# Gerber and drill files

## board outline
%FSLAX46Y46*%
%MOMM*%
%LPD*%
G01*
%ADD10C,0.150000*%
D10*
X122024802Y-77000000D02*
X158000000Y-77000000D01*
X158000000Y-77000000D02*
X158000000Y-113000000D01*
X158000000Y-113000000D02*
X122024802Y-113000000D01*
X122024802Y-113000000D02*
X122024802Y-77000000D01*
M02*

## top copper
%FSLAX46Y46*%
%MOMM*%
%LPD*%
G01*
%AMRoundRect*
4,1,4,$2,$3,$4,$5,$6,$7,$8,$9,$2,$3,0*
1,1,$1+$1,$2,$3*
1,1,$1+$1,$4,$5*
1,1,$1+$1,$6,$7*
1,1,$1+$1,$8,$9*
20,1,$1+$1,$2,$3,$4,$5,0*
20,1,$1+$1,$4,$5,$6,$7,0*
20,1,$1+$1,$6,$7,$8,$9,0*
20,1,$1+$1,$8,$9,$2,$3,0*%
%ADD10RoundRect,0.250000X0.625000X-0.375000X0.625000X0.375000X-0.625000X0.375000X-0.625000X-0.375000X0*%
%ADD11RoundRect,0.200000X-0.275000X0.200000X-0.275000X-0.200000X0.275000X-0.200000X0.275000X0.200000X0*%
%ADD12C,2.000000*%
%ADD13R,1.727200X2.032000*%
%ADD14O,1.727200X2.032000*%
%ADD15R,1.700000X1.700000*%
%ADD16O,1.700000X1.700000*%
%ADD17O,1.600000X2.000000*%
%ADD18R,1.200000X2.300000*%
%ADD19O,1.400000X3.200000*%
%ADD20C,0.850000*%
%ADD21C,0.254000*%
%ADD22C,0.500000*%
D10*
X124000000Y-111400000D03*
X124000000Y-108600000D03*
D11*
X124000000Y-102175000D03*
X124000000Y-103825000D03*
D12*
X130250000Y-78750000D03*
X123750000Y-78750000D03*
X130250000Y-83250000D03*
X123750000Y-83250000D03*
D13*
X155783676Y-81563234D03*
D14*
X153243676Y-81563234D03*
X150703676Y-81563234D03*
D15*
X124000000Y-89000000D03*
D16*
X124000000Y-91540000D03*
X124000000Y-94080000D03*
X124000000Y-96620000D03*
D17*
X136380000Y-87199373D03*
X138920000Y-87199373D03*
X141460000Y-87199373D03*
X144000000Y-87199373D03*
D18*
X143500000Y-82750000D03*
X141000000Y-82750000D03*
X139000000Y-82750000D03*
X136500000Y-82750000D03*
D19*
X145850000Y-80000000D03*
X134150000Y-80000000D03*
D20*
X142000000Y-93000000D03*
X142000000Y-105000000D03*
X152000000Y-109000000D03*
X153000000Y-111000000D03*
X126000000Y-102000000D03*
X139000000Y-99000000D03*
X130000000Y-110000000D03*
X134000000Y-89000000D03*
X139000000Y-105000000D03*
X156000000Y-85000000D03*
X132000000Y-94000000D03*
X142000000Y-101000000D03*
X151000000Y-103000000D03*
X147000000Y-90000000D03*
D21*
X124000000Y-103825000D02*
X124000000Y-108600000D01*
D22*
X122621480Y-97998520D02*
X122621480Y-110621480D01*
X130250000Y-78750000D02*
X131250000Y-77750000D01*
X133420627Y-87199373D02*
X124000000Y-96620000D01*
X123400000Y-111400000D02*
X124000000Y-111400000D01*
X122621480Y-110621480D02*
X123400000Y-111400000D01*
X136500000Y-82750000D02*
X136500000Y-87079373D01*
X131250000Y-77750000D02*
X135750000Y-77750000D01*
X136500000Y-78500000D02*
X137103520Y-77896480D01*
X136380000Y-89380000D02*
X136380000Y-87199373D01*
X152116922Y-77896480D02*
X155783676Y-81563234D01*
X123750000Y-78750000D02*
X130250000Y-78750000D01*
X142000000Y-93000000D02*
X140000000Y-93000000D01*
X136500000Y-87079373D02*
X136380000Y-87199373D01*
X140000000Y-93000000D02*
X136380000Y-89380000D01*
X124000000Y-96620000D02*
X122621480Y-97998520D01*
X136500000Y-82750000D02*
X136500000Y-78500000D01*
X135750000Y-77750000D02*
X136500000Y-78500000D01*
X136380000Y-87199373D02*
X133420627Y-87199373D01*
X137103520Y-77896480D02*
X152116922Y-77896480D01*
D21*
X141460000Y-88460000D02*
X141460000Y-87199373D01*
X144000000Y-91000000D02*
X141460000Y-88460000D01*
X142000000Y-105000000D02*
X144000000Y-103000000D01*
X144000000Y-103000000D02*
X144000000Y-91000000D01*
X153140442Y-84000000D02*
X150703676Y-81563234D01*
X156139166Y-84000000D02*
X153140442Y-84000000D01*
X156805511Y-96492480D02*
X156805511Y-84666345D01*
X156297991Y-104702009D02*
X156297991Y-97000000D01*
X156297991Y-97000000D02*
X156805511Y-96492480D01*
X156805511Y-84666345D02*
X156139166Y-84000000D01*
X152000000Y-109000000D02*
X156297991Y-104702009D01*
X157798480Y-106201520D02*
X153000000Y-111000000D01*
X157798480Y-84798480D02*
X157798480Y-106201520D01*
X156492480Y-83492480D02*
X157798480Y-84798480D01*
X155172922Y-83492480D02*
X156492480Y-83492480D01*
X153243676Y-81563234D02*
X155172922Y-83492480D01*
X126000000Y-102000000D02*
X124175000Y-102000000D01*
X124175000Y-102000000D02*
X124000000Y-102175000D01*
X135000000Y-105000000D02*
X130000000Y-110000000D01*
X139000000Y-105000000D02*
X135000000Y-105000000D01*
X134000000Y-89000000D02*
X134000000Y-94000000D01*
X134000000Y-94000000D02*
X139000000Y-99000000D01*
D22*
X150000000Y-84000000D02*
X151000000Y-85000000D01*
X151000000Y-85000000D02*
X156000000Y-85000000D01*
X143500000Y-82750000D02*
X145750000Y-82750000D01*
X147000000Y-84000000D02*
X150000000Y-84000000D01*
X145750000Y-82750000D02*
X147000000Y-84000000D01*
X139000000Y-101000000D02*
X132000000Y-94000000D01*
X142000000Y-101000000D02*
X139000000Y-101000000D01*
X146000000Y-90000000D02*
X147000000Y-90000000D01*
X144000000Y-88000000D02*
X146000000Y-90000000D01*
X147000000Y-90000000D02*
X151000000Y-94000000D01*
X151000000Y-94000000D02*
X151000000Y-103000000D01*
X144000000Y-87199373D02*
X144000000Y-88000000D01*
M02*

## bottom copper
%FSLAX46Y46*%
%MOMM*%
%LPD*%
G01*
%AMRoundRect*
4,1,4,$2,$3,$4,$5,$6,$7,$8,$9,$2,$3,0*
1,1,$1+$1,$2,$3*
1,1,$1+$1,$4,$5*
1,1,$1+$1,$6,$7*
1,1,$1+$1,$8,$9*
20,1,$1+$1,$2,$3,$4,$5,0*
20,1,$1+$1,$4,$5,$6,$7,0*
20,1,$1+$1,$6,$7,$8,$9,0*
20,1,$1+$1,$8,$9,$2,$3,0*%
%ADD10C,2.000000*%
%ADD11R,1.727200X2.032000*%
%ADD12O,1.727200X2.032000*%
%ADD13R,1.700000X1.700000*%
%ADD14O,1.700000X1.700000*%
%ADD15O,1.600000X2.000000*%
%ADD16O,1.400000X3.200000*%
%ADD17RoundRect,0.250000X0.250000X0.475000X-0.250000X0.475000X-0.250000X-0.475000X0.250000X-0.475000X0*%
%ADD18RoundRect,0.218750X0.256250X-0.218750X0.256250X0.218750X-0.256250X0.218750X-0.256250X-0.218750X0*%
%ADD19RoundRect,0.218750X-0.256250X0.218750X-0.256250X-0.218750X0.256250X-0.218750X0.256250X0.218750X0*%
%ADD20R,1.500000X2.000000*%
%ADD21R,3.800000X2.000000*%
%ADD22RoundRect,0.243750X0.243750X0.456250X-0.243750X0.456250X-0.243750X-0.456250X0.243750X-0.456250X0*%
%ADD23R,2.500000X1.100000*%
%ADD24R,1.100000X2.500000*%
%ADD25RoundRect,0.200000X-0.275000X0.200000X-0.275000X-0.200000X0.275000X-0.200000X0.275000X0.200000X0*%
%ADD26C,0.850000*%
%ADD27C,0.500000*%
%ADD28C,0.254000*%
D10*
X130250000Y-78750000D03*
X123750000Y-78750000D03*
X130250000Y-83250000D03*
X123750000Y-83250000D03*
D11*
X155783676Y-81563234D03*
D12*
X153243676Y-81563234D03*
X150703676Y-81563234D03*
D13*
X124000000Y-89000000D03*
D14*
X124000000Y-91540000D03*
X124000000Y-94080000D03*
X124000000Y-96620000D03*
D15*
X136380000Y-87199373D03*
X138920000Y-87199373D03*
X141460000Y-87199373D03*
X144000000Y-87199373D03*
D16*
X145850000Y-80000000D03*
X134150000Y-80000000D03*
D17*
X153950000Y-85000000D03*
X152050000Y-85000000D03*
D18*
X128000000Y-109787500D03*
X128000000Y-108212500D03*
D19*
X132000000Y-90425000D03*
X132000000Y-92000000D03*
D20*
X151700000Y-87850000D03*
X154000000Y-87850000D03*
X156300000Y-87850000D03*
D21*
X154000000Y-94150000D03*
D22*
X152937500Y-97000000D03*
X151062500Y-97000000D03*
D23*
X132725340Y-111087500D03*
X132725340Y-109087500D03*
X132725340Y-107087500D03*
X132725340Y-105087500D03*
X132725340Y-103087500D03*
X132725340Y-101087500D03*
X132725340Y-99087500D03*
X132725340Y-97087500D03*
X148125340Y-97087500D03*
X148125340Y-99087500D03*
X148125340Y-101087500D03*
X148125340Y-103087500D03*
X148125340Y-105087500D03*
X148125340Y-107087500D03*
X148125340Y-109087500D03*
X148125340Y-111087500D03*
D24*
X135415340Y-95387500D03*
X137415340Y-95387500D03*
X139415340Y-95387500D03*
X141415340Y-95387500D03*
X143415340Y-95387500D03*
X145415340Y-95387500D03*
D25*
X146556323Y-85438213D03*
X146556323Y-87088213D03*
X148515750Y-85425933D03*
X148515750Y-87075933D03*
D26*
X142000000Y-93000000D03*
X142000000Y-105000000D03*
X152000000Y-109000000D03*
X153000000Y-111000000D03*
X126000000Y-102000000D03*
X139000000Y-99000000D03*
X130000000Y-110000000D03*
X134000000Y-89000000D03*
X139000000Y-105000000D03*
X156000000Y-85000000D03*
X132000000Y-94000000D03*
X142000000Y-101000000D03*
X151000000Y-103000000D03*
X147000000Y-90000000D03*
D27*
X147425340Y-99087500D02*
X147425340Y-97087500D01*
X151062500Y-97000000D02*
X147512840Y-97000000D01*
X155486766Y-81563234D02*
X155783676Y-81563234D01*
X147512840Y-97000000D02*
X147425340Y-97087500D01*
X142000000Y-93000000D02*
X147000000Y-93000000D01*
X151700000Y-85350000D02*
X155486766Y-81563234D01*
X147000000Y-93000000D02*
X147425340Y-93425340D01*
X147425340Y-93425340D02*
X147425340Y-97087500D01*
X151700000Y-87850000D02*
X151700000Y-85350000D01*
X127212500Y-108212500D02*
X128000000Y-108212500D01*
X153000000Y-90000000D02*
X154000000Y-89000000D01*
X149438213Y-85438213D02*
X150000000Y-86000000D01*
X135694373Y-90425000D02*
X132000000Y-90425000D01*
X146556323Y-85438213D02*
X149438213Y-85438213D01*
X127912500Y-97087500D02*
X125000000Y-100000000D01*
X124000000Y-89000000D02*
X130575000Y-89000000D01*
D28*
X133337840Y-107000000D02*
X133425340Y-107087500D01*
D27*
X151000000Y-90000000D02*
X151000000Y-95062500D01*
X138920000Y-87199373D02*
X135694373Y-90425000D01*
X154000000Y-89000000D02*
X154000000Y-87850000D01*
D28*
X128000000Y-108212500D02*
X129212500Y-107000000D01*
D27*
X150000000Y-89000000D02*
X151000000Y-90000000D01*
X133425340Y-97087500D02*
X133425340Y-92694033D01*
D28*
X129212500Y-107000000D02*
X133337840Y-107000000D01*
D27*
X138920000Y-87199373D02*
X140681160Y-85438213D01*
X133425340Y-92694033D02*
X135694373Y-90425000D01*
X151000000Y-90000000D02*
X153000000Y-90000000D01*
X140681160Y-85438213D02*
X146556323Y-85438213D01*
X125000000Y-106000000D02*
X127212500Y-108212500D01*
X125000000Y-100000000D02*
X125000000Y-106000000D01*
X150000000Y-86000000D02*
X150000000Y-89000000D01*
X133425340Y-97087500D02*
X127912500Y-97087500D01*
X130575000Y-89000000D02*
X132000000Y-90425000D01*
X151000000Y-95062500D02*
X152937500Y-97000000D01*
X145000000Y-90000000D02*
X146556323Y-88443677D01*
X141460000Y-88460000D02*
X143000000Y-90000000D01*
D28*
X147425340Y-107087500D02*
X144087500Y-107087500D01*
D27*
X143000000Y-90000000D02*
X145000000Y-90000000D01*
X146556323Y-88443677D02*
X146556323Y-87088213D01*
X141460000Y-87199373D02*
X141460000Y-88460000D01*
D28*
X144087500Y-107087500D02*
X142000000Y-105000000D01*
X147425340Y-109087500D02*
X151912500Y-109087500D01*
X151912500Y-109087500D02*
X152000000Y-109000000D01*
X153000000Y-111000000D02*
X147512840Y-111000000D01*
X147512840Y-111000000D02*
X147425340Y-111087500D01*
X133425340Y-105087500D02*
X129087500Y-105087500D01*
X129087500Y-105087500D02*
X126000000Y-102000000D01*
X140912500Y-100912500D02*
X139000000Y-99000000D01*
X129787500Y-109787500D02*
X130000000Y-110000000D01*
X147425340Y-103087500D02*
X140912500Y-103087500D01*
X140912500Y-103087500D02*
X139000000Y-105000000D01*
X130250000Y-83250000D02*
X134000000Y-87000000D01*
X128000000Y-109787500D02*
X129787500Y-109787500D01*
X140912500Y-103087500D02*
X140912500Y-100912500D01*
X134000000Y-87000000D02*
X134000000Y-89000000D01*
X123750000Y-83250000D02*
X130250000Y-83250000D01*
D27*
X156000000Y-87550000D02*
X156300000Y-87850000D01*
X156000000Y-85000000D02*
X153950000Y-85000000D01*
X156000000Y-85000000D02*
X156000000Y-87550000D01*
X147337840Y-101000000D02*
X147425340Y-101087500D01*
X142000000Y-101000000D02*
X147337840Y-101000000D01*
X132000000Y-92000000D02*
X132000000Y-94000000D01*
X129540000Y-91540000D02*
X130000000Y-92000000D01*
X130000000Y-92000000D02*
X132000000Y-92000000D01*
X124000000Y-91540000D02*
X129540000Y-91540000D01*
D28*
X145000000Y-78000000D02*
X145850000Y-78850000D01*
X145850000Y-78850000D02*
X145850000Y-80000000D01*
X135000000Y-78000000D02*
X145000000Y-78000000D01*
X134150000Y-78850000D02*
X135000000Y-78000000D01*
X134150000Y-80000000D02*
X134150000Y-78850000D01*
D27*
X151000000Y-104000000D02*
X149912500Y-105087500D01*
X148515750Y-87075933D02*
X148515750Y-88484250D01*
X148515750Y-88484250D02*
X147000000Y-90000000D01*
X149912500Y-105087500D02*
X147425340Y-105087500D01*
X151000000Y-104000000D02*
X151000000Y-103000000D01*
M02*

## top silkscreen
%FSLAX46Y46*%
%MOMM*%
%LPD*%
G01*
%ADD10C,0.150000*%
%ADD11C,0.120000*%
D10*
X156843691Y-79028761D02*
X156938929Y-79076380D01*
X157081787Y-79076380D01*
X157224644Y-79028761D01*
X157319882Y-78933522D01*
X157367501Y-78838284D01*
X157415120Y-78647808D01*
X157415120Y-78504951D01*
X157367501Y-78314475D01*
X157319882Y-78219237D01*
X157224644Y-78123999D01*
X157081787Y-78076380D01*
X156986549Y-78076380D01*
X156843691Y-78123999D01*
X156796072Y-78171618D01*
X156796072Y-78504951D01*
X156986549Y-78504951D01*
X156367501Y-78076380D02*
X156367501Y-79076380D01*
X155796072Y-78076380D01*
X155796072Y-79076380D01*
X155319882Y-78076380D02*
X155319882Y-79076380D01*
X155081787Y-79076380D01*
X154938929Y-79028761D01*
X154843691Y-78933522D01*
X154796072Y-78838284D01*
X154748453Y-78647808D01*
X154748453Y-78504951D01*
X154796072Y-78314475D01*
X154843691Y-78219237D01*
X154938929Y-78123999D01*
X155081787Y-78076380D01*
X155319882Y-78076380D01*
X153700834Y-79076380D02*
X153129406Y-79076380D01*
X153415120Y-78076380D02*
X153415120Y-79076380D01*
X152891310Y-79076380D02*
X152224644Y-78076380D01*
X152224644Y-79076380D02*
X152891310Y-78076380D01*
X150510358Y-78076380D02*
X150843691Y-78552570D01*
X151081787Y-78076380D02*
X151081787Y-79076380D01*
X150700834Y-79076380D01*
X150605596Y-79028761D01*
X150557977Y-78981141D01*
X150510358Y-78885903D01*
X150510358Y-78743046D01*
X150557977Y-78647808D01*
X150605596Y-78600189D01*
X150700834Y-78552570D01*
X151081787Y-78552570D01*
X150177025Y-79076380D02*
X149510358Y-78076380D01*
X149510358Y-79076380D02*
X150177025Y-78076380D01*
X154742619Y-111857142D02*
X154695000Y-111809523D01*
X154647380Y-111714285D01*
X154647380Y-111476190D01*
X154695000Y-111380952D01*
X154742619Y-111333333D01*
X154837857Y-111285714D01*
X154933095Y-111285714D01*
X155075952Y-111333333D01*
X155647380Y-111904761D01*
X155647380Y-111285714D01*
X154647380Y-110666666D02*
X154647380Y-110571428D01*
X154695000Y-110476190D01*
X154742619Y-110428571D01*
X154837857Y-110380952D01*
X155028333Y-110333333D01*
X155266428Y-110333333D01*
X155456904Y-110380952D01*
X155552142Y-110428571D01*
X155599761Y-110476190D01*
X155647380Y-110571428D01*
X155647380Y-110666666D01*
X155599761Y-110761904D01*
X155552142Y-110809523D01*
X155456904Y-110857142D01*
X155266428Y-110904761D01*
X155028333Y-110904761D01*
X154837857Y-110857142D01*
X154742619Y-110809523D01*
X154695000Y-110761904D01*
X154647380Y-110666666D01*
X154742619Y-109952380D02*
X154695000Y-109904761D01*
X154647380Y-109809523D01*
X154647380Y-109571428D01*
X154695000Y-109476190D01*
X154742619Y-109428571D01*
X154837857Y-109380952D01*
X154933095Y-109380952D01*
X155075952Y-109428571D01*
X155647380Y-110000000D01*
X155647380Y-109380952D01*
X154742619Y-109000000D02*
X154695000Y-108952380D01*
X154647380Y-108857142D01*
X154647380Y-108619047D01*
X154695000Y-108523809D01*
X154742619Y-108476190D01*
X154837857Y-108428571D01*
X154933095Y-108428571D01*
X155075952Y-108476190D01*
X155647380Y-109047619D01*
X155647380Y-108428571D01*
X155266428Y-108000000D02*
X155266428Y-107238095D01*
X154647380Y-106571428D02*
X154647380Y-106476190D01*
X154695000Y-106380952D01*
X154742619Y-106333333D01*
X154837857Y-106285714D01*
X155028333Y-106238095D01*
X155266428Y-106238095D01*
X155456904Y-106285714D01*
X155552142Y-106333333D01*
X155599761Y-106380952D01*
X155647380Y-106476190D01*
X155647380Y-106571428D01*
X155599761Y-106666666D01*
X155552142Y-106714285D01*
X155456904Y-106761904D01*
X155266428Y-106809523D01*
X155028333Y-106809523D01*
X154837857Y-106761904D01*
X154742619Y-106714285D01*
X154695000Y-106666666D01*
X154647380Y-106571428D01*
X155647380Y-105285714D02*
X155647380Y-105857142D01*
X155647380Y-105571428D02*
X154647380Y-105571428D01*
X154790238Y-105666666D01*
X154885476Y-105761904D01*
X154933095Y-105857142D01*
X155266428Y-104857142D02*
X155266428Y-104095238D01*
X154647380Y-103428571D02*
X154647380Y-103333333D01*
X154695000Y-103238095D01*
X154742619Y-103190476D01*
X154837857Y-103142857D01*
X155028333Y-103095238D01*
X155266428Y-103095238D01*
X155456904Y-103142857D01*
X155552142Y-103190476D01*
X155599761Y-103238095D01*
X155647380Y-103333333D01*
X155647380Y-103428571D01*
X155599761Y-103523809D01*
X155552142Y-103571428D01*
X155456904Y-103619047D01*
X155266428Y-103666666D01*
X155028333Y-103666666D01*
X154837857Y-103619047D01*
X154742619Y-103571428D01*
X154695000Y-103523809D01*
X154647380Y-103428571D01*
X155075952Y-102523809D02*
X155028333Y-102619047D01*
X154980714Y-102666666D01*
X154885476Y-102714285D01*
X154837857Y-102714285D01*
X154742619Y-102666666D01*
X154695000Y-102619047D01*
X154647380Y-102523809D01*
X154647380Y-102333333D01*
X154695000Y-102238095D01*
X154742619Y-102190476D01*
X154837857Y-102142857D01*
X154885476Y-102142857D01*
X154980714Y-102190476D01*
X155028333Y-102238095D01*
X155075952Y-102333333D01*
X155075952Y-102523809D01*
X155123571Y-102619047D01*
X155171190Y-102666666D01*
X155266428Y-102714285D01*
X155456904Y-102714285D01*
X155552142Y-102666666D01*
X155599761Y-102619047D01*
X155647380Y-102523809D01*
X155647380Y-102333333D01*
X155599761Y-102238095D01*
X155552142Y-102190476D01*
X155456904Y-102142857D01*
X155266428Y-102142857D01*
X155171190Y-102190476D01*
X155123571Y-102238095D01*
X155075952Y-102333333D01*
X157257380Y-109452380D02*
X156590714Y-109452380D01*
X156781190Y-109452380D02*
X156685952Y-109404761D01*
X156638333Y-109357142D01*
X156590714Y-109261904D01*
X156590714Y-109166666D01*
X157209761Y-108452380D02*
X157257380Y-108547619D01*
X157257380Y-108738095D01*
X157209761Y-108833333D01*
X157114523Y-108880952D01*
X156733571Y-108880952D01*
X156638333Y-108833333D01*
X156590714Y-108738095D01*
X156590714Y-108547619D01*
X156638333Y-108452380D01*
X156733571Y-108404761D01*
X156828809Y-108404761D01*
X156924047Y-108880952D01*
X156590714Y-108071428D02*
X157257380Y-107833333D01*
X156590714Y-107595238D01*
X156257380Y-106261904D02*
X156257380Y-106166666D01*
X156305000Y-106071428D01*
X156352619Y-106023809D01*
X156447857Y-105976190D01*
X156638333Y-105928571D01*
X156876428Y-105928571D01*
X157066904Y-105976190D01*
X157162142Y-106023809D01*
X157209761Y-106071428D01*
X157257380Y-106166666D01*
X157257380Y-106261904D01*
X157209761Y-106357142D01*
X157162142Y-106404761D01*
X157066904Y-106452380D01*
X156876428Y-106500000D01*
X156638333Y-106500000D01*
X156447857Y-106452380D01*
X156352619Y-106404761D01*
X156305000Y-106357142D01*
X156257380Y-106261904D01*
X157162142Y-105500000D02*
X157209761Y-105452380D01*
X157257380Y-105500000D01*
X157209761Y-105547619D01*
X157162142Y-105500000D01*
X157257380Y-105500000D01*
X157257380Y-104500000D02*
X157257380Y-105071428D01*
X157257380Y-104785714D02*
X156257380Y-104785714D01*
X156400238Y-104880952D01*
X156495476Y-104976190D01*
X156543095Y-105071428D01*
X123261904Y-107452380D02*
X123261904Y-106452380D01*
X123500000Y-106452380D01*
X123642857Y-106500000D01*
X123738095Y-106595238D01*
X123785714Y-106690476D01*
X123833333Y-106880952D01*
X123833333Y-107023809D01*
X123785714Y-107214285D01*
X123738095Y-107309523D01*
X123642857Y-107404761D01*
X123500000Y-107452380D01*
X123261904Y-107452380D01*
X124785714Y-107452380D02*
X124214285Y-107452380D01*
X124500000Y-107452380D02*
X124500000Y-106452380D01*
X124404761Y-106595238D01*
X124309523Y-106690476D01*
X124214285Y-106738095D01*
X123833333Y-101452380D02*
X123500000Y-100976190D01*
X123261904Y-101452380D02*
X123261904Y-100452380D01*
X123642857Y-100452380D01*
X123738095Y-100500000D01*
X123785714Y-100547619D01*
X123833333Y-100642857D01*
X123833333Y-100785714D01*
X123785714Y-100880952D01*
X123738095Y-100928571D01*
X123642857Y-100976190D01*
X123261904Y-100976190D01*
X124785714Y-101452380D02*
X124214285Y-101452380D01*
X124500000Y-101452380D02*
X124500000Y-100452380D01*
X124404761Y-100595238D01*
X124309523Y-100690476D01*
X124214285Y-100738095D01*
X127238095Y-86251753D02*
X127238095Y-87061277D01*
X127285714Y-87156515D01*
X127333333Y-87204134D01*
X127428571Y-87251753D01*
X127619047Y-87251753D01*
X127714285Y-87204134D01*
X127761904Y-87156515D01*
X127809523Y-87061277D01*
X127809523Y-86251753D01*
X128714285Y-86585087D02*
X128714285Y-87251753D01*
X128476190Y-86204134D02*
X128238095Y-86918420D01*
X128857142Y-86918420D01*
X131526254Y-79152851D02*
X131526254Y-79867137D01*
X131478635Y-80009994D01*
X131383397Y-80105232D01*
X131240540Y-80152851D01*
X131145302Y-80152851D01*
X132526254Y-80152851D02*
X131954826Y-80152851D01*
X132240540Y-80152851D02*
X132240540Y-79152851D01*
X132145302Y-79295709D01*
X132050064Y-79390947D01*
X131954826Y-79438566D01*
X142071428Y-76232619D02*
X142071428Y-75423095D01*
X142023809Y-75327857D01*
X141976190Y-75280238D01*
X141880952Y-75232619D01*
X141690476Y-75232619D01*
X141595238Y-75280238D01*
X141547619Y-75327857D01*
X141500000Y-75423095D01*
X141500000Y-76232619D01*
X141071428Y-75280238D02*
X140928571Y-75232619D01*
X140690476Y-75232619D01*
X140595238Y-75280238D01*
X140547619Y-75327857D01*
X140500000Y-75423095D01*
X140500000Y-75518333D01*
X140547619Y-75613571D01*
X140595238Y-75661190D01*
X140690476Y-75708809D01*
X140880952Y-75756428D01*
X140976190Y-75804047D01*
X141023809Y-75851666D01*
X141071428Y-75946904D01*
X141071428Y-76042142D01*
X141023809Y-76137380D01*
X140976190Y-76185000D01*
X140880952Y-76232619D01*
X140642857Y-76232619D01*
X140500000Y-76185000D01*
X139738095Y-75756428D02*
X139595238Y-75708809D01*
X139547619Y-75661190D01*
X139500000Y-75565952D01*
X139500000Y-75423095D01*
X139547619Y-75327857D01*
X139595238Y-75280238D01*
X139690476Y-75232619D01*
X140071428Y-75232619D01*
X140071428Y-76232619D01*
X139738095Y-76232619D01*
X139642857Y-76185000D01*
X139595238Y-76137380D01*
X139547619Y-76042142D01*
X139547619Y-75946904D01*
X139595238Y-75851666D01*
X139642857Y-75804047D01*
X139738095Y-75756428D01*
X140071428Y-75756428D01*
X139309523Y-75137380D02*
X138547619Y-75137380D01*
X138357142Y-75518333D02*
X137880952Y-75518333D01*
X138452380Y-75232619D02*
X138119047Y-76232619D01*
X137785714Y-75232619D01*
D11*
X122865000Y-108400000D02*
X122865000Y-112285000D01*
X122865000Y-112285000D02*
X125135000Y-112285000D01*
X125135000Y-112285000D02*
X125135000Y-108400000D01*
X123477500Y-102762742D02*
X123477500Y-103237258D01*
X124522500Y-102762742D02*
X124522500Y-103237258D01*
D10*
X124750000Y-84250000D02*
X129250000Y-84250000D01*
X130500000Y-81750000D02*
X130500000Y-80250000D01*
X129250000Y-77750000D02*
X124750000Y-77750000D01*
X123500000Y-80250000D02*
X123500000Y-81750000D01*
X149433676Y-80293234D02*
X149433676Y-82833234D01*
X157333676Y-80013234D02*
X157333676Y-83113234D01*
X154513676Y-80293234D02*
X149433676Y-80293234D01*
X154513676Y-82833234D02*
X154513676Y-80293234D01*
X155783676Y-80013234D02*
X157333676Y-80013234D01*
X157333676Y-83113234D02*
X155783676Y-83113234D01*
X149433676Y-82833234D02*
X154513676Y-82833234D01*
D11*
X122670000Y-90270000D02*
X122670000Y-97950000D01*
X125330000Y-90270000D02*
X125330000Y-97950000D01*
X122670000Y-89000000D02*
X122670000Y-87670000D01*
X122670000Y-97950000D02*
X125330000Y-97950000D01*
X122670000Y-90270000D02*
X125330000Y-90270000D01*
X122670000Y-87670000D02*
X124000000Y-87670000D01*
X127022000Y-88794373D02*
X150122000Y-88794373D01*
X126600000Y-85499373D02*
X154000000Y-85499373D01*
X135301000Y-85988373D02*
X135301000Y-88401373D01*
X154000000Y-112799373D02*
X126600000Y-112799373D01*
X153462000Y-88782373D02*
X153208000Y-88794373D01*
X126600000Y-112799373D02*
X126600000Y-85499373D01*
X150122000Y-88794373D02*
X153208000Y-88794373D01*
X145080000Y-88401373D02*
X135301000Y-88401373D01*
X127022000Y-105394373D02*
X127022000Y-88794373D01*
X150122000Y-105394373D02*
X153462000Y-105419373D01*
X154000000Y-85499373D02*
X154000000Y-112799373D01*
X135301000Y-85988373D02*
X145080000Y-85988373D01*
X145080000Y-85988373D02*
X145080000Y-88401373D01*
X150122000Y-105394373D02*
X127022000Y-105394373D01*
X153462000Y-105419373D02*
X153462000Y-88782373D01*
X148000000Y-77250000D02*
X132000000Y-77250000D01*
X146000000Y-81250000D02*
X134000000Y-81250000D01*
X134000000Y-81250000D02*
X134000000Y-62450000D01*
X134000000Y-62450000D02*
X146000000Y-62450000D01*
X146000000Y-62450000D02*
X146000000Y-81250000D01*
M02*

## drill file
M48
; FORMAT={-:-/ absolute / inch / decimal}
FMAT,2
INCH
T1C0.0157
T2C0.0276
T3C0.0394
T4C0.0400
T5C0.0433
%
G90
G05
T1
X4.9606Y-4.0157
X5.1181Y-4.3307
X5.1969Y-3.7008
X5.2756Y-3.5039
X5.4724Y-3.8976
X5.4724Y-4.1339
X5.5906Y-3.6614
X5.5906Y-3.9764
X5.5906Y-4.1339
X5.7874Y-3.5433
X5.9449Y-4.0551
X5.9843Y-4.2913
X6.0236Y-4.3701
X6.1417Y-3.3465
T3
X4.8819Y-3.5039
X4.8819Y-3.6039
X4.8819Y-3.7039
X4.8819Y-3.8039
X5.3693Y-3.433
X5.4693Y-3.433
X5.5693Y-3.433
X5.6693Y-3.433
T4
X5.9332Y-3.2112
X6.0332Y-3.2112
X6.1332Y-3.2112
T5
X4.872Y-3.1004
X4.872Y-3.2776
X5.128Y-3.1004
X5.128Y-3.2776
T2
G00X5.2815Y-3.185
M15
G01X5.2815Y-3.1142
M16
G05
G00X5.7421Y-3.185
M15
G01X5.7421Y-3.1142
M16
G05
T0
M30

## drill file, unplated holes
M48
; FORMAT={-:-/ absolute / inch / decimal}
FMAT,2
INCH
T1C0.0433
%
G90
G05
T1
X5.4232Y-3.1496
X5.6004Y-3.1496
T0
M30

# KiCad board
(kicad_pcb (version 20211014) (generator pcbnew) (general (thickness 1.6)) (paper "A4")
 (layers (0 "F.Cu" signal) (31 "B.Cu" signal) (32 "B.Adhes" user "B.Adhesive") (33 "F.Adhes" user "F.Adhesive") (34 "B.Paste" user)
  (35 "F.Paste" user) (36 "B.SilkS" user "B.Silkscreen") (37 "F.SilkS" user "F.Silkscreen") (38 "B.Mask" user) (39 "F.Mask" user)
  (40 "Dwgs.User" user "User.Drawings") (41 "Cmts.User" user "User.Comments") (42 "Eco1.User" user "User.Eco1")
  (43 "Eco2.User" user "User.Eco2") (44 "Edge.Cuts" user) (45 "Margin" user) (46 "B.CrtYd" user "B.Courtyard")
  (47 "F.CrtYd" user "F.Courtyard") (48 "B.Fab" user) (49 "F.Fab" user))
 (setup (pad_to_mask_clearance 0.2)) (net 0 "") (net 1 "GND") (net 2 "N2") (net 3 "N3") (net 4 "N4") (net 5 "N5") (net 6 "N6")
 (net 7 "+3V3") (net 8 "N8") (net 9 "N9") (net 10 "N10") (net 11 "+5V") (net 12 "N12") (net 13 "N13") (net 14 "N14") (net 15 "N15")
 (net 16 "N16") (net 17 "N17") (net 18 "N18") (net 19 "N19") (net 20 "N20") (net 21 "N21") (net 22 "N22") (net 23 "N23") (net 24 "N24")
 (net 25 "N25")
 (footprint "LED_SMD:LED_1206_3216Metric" (layer "F.Cu") (at 124 110 90)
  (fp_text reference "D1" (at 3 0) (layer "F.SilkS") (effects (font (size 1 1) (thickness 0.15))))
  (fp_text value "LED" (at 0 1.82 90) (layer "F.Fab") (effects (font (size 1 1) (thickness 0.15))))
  (fp_line (start 1.6 -1.135) (end -2.285 -1.135) (layer "F.SilkS") (width 0.12))
  (fp_line (start -2.285 -1.135) (end -2.285 1.135) (layer "F.SilkS") (width 0.12))
  (fp_line (start -2.285 1.135) (end 1.6 1.135) (layer "F.SilkS") (width 0.12))
  (pad "1" smd roundrect locked (at -1.4 0 90) (size 1.25 1.75) (layers "F.Cu" "F.Paste" "F.Mask") (roundrect_rratio 0.2) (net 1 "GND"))
  (pad "2" smd roundrect locked (at 1.4 0 90) (size 1.25 1.75) (layers "F.Cu" "F.Paste" "F.Mask") (roundrect_rratio 0.2) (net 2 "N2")))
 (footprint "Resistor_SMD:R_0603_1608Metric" (layer "F.Cu") (at 124 103 -90)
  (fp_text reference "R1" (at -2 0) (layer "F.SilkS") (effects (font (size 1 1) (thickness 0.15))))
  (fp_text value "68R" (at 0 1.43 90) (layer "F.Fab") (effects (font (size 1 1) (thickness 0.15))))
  (fp_line (start -0.237258 0.5225) (end 0.237258 0.5225) (layer "F.SilkS") (width 0.12))
  (fp_line (start -0.237258 -0.5225) (end 0.237258 -0.5225) (layer "F.SilkS") (width 0.12))
  (pad "1" smd roundrect locked (at -0.825 0 270) (size 0.8 0.95) (layers "F.Cu" "F.Paste" "F.Mask") (roundrect_rratio 0.25) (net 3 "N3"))
  (pad "2" smd roundrect locked (at 0.825 0 270) (size 0.8 0.95) (layers "F.Cu" "F.Paste" "F.Mask") (roundrect_rratio 0.25) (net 2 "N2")))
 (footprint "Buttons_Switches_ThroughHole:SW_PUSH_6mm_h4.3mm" (layer "F.Cu") (at 123.75 78.75)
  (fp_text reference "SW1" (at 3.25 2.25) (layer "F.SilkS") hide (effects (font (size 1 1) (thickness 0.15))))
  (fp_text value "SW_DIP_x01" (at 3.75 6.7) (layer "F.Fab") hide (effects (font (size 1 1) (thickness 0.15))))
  (fp_line (start 1 5.5) (end 5.5 5.5) (layer "F.SilkS") (width 0.15))
  (fp_line (start 6.75 3) (end 6.75 1.5) (layer "F.SilkS") (width 0.15))
  (fp_line (start 5.5 -1) (end 1 -1) (layer "F.SilkS") (width 0.15))
  (fp_line (start -0.25 1.5) (end -0.25 3) (layer "F.SilkS") (width 0.15))
  (pad "1" thru_hole circle locked (at 6.5 0 90) (size 2 2) (drill 1.1) (layers *.Cu *.Mask) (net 1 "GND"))
  (pad "1" thru_hole circle locked (at 0 0 90) (size 2 2) (drill 1.1) (layers *.Cu *.Mask) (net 1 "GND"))
  (pad "2" thru_hole circle locked (at 6.5 4.5 90) (size 2 2) (drill 1.1) (layers *.Cu *.Mask) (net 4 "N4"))
  (pad "2" thru_hole circle locked (at 0 4.5 90) (size 2 2) (drill 1.1) (layers *.Cu *.Mask) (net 4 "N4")))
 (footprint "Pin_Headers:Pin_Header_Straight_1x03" (layer "F.Cu") (at 155.783676 81.563234 -90)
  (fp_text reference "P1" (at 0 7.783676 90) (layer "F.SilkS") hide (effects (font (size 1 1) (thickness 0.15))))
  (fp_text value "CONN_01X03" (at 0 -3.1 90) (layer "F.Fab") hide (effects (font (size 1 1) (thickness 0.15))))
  (fp_line (start -1.27 6.35) (end 1.27 6.35) (layer "F.SilkS") (width 0.15))
  (fp_line (start -1.55 -1.55) (end 1.55 -1.55) (layer "F.SilkS") (width 0.15))
  (fp_line (start -1.27 1.27) (end -1.27 6.35) (layer "F.SilkS") (width 0.15))
  (fp_line (start 1.27 1.27) (end -1.27 1.27) (layer "F.SilkS") (width 0.15))
  (fp_line (start -1.55 0) (end -1.55 -1.55) (layer "F.SilkS") (width 0.15))
  (fp_line (start 1.55 -1.55) (end 1.55 0) (layer "F.SilkS") (width 0.15))
  (fp_line (start 1.27 6.35) (end 1.27 1.27) (layer "F.SilkS") (width 0.15))
  (pad "1" thru_hole rect locked (at 0 0 270) (size 2.032 1.7272) (drill 1.016) (layers *.Cu *.Mask) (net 1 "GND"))
  (pad "2" thru_hole oval locked (at 0 2.54 270) (size 2.032 1.7272) (drill 1.016) (layers *.Cu *.Mask) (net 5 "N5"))
  (pad "3" thru_hole oval locked (at 0 5.08 270) (size 2.032 1.7272) (drill 1.016) (layers *.Cu *.Mask) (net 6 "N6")))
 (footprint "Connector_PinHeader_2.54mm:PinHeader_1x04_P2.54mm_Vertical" (layer "F.Cu") (at 124 89)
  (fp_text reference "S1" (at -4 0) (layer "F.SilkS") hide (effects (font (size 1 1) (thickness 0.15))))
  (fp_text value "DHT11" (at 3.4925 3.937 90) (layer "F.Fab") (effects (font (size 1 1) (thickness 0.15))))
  (fp_line (start -1.33 1.27) (end -1.33 8.95) (layer "F.SilkS") (width 0.12))
  (fp_line (start 1.33 1.27) (end 1.33 8.95) (layer "F.SilkS") (width 0.12))
  (fp_line (start -1.33 0) (end -1.33 -1.33) (layer "F.SilkS") (width 0.12))
  (fp_line (start -1.33 8.95) (end 1.33 8.95) (layer "F.SilkS") (width 0.12))
  (fp_line (start -1.33 1.27) (end 1.33 1.27) (layer "F.SilkS") (width 0.12))
  (fp_line (start -1.33 -1.33) (end 0 -1.33) (layer "F.SilkS") (width 0.12))
  (pad "1" thru_hole rect locked (at 0 0) (size 1.7 1.7) (drill 1) (layers *.Cu *.Mask) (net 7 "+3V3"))
  (pad "2" thru_hole oval locked (at 0 2.54) (size 1.7 1.7) (drill 1) (layers *.Cu *.Mask) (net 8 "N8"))
  (pad "3" thru_hole oval locked (at 0 5.08) (size 1.7 1.7) (drill 1) (layers *.Cu *.Mask))
  (pad "4" thru_hole oval locked (at 0 7.62) (size 1.7 1.7) (drill 1) (layers *.Cu *.Mask) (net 1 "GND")))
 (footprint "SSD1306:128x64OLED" (layer "F.Cu") (at 140 97.799373)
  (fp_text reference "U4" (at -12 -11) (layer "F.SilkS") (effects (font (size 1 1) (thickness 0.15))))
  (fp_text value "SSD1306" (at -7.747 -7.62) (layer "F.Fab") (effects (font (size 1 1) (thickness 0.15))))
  (fp_line (start -12.978 -9.005) (end 10.122 -9.005) (layer "F.SilkS") (width 0.12))
  (fp_line (start -13.4 -12.3) (end 14 -12.3) (layer "F.SilkS") (width 0.12))
  (fp_line (start -4.699 -11.811) (end -4.699 -9.398) (layer "F.SilkS") (width 0.12))
  (fp_line (start 14 15) (end -13.4 15) (layer "F.SilkS") (width 0.12))
  (fp_line (start 13.462 -9.017) (end 13.208 -9.005) (layer "F.SilkS") (width 0.12))
  (fp_line (start -13.4 15) (end -13.4 -12.3) (layer "F.SilkS") (width 0.12))
  (fp_line (start 10.122 -9.005) (end 13.208 -9.005) (layer "F.SilkS") (width 0.12))
  (fp_line (start 5.08 -9.398) (end -4.699 -9.398) (layer "F.SilkS") (width 0.12))
  (fp_line (start -12.978 7.595) (end -12.978 -9.005) (layer "F.SilkS") (width 0.12))
  (fp_line (start 10.122 7.595) (end 13.462 7.62) (layer "F.SilkS") (width 0.12))
  (fp_line (start 14 -12.3) (end 14 15) (layer "F.SilkS") (width 0.12))
  (fp_line (start -4.699 -11.811) (end 5.08 -11.811) (layer "F.SilkS") (width 0.12))
  (fp_line (start 5.08 -11.811) (end 5.08 -9.398) (layer "F.SilkS") (width 0.12))
  (fp_line (start 10.122 7.595) (end -12.978 7.595) (layer "F.SilkS") (width 0.12))
  (fp_line (start 13.462 7.62) (end 13.462 -9.017) (layer "F.SilkS") (width 0.12))
  (pad "1" thru_hole oval locked (at -3.62 -10.6 90) (size 2 1.6) (drill 1) (layers *.Cu *.Mask) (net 1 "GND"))
  (pad "2" thru_hole oval locked (at -1.08 -10.6 90) (size 2 1.6) (drill 1) (layers *.Cu *.Mask) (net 7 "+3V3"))
  (pad "3" thru_hole oval locked (at 1.46 -10.6 90) (size 2 1.6) (drill 1) (layers *.Cu *.Mask) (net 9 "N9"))
  (pad "4" thru_hole oval locked (at 4 -10.6 90) (size 2 1.6) (drill 1) (layers *.Cu *.Mask) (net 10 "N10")))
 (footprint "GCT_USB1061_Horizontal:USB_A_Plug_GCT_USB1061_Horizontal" (layer "F.Cu") (at 140 80 180)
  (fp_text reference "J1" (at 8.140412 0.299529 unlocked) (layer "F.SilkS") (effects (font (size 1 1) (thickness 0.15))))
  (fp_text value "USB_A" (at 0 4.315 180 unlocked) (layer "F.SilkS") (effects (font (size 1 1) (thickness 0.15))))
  (fp_line (start -8 2.75) (end 8 2.75) (layer "F.SilkS") (width 0.12))
  (fp_rect (start -6 -1.25) (end 6 17.55) (layer "F.SilkS") (width 0.12) (fill none))
  (pad "" np_thru_hole circle (at 2.25 0 180) (size 1.1 1.1) (drill 1.1) (layers *.Mask))
  (pad "" np_thru_hole circle (at -2.25 0 180) (size 1.1 1.1) (drill 1.1) (layers *.Mask))
  (pad "1" smd rect (at -3.5 -2.75 180) (size 1.2 2.3) (layers "F.Cu" "F.Paste" "F.Mask") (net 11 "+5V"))
  (pad "2" smd rect (at -1 -2.75 180) (size 1.2 2.3) (layers "F.Cu" "F.Paste" "F.Mask") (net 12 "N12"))
  (pad "3" smd rect (at 1 -2.75 180) (size 1.2 2.3) (layers "F.Cu" "F.Paste" "F.Mask") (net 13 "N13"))
  (pad "4" smd rect (at 3.5 -2.75 180) (size 1.2 2.3) (layers "F.Cu" "F.Paste" "F.Mask") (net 1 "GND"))
  (pad "5" thru_hole oval (at -5.85 0 180) (size 1.4 3.2) (drill oval 0.7 2.5) (layers *.Cu *.Mask) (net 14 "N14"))
  (pad "5" thru_hole oval (at 5.85 0 180) (size 1.4 3.2) (drill oval 0.7 2.5) (layers *.Cu *.Mask) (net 14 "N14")))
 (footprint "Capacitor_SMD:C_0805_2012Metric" (layer "B.Cu") (at 153 85 180)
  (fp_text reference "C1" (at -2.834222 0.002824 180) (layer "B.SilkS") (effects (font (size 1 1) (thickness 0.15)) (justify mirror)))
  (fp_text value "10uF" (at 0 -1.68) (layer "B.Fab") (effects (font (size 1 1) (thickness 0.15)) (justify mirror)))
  (pad "1" smd roundrect locked (at -0.95 0 180) (size 1 1.45) (layers "B.Cu" "B.Paste" "B.Mask") (roundrect_rratio 0.25) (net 11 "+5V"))
  (pad "2" smd roundrect locked (at 0.95 0 180) (size 1 1.45) (layers "B.Cu" "B.Paste" "B.Mask") (roundrect_rratio 0.25) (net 1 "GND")))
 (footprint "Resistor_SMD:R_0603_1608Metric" (layer "B.Cu") (at 128 109 90)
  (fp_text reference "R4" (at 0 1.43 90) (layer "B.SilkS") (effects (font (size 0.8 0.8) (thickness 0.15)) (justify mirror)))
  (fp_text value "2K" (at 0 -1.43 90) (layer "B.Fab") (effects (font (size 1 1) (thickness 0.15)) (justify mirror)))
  (pad "1" smd roundrect locked (at -0.7875 0 90) (size 0.875 0.95) (layers "B.Cu" "B.Paste" "B.Mask") (roundrect_rratio 0.25) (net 4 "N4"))
  (pad "2" smd roundrect locked (at 0.7875 0 90) (size 0.875 0.95) (layers "B.Cu" "B.Paste" "B.Mask") (roundrect_rratio 0.25) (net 7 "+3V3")))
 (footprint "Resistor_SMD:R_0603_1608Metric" (layer "B.Cu") (at 132 91.2125 -90)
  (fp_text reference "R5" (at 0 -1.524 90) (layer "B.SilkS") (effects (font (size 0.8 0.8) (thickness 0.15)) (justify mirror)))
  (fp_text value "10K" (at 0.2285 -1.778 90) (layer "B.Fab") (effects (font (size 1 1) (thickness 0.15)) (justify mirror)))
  (pad "1" smd roundrect locked (at -0.7875 0 270) (size 0.875 0.95) (layers "B.Cu" "B.Paste" "B.Mask") (roundrect_rratio 0.25)
   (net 7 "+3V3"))
  (pad "2" smd roundrect locked (at 0.7875 0 270) (size 0.875 0.95) (layers "B.Cu" "B.Paste" "B.Mask") (roundrect_rratio 0.25) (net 8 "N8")))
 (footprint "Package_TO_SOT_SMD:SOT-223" (layer "B.Cu") (at 154 91 -90)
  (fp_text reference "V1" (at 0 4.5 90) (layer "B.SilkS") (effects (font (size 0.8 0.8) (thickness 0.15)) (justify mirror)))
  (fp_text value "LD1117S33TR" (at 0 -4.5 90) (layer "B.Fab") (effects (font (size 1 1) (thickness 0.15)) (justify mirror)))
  (pad "1" smd rect locked (at -3.15 2.3 270) (size 2 1.5) (layers "B.Cu" "B.Paste" "B.Mask") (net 1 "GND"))
  (pad "2" smd rect locked (at -3.15 0 270) (size 2 1.5) (layers "B.Cu" "B.Paste" "B.Mask") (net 7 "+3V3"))
  (pad "3" smd rect locked (at -3.15 -2.3 270) (size 2 1.5) (layers "B.Cu" "B.Paste" "B.Mask") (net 11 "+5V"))
  (pad "4" smd rect locked (at 3.15 0 270) (size 2 3.8) (layers "B.Cu" "B.Paste" "B.Mask")))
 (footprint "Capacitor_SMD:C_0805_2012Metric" (layer "B.Cu") (at 152 97 180)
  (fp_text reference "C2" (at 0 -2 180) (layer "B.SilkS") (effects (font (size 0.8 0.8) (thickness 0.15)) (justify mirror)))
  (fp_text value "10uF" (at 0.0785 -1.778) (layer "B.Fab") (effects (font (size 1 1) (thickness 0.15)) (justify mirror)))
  (pad "1" smd roundrect locked (at -0.9375 0 180) (size 0.975 1.4) (layers "B.Cu" "B.Paste" "B.Mask") (roundrect_rratio 0.25)
   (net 7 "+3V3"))
  (pad "2" smd roundrect locked (at 0.9375 0 180) (size 0.975 1.4) (layers "B.Cu" "B.Paste" "B.Mask") (roundrect_rratio 0.25) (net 1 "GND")))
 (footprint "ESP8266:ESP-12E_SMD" (layer "B.Cu") (at 133.42534 111.0875)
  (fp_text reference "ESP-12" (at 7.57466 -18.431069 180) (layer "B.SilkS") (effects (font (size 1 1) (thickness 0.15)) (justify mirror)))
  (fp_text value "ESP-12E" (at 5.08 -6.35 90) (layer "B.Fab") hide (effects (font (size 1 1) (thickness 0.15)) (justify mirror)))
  (pad "1" smd rect locked (at 0 0) (size 2.5 1.1) (drill (offset -0.7 0)) (layers "B.Cu" "B.Paste" "B.Mask") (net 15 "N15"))
  (pad "2" smd rect locked (at 0 -2) (size 2.5 1.1) (drill (offset -0.7 0)) (layers "B.Cu" "B.Paste" "B.Mask") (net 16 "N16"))
  (pad "3" smd rect locked (at 0 -4) (size 2.5 1.1) (drill (offset -0.7 0)) (layers "B.Cu" "B.Paste" "B.Mask") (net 7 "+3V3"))
  (pad "4" smd rect locked (at 0 -6) (size 2.5 1.1) (drill (offset -0.7 0)) (layers "B.Cu" "B.Paste" "B.Mask") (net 3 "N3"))
  (pad "5" smd rect locked (at 0 -8) (size 2.5 1.1) (drill (offset -0.7 0)) (layers "B.Cu" "B.Paste" "B.Mask") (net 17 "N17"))
  (pad "6" smd rect locked (at 0 -10) (size 2.5 1.1) (drill (offset -0.7 0)) (layers "B.Cu" "B.Paste" "B.Mask") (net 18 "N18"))
  (pad "7" smd rect locked (at 0 -12) (size 2.5 1.1) (drill (offset -0.7 0)) (layers "B.Cu" "B.Paste" "B.Mask") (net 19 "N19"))
  (pad "8" smd rect locked (at 0 -14) (size 2.5 1.1) (drill (offset -0.7 0)) (layers "B.Cu" "B.Paste" "B.Mask") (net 7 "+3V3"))
  (pad "9" smd rect locked (at 14 -14) (size 2.5 1.1) (drill (offset 0.7 0)) (layers "B.Cu" "B.Paste" "B.Mask") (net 1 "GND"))
  (pad "10" smd rect locked (at 14 -12) (size 2.5 1.1) (drill (offset 0.7 0)) (layers "B.Cu" "B.Paste" "B.Mask") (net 1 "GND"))
  (pad "11" smd rect locked (at 14 -10) (size 2.5 1.1) (drill (offset 0.7 0)) (layers "B.Cu" "B.Paste" "B.Mask") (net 8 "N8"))
  (pad "12" smd rect locked (at 14 -8) (size 2.5 1.1) (drill (offset 0.7 0)) (layers "B.Cu" "B.Paste" "B.Mask") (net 4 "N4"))
  (pad "13" smd rect locked (at 14 -6) (size 2.5 1.1) (drill (offset 0.7 0)) (layers "B.Cu" "B.Paste" "B.Mask") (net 10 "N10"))
  (pad "14" smd rect locked (at 14 -4) (size 2.5 1.1) (drill (offset 0.7 0)) (layers "B.Cu" "B.Paste" "B.Mask") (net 9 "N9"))
  (pad "15" smd rect locked (at 14 -2) (size 2.5 1.1) (drill (offset 0.7 0)) (layers "B.Cu" "B.Paste" "B.Mask") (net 6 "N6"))
  (pad "16" smd rect locked (at 14 0) (size 2.5 1.1) (drill (offset 0.7 0)) (layers "B.Cu" "B.Paste" "B.Mask") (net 5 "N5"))
  (pad "17" smd rect locked (at 1.99 -15 270) (size 2.5 1.1) (drill (offset -0.7 0)) (layers "B.Cu" "B.Paste" "B.Mask") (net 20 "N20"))
  (pad "18" smd rect locked (at 3.99 -15 270) (size 2.5 1.1) (drill (offset -0.7 0)) (layers "B.Cu" "B.Paste" "B.Mask") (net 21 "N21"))
  (pad "19" smd rect locked (at 5.99 -15 270) (size 2.5 1.1) (drill (offset -0.7 0)) (layers "B.Cu" "B.Paste" "B.Mask") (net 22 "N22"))
  (pad "20" smd rect locked (at 7.99 -15 270) (size 2.5 1.1) (drill (offset -0.7 0)) (layers "B.Cu" "B.Paste" "B.Mask") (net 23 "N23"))
  (pad "21" smd rect locked (at 9.99 -15 270) (size 2.5 1.1) (drill (offset -0.7 0)) (layers "B.Cu" "B.Paste" "B.Mask") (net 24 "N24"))
  (pad "22" smd rect locked (at 11.99 -15 270) (size 2.5 1.1) (drill (offset -0.7 0)) (layers "B.Cu" "B.Paste" "B.Mask") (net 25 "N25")))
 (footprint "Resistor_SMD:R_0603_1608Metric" (layer "B.Cu") (at 146.556323 86.263213 -90)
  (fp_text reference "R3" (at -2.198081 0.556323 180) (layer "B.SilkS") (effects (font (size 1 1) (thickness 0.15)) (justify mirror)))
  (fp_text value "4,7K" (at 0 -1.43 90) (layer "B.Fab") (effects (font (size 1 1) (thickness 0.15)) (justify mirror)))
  (pad "1" smd roundrect locked (at -0.825 0 270) (size 0.8 0.95) (layers "B.Cu" "B.Paste" "B.Mask") (roundrect_rratio 0.25) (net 7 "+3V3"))
  (pad "2" smd roundrect locked (at 0.825 0 270) (size 0.8 0.95) (layers "B.Cu" "B.Paste" "B.Mask") (roundrect_rratio 0.25) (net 9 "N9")))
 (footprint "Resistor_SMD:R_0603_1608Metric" (layer "B.Cu") (at 148.51575 86.250933 -90)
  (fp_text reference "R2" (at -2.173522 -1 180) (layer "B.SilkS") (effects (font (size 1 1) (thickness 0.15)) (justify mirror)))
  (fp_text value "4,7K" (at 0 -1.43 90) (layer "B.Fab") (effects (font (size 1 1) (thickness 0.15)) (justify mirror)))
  (pad "1" smd roundrect locked (at -0.825 0 270) (size 0.8 0.95) (layers "B.Cu" "B.Paste" "B.Mask") (roundrect_rratio 0.25) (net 7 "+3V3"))
  (pad "2" smd roundrect locked (at 0.825 0 270) (size 0.8 0.95) (layers "B.Cu" "B.Paste" "B.Mask") (roundrect_rratio 0.25) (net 10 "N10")))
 (gr_rect (start 122.024802 77) (end 158 113) (layer "Edge.Cuts") (width 0.15) (fill none))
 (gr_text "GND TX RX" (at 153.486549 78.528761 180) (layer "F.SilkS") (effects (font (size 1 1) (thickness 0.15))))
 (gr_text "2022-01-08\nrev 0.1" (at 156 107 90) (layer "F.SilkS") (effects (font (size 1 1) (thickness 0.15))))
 (segment (start 124 103.825) (end 124 108.6) (width 0.254) (layer "F.Cu") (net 2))
 (segment (start 122.62148 97.99852) (end 122.62148 110.62148) (width 0.5) (layer "F.Cu") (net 1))
 (segment (start 130.25 78.75) (end 131.25 77.75) (width 0.5) (layer "F.Cu") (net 1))
 (segment (start 133.420627 87.199373) (end 124 96.62) (width 0.5) (layer "F.Cu") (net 1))
 (segment (start 123.4 111.4) (end 124 111.4) (width 0.5) (layer "F.Cu") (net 1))
 (segment (start 122.62148 110.62148) (end 123.4 111.4) (width 0.5) (layer "F.Cu") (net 1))
 (segment (start 136.5 82.75) (end 136.5 87.079373) (width 0.5) (layer "F.Cu") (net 1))
 (segment (start 131.25 77.75) (end 135.75 77.75) (width 0.5) (layer "F.Cu") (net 1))
 (segment (start 136.5 78.5) (end 137.10352 77.89648) (width 0.5) (layer "F.Cu") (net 1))
 (segment (start 136.38 89.38) (end 136.38 87.199373) (width 0.5) (layer "F.Cu") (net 1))
 (segment (start 152.116922 77.89648) (end 155.783676 81.563234) (width 0.5) (layer "F.Cu") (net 1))
 (segment (start 123.75 78.75) (end 130.25 78.75) (width 0.5) (layer "F.Cu") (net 1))
 (segment (start 142 93) (end 140 93) (width 0.5) (layer "F.Cu") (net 1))
 (segment (start 136.5 87.079373) (end 136.38 87.199373) (width 0.5) (layer "F.Cu") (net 1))
 (segment (start 140 93) (end 136.38 89.38) (width 0.5) (layer "F.Cu") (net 1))
 (segment (start 124 96.62) (end 122.62148 97.99852) (width 0.5) (layer "F.Cu") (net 1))
 (segment (start 136.5 82.75) (end 136.5 78.5) (width 0.5) (layer "F.Cu") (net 1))
 (segment (start 135.75 77.75) (end 136.5 78.5) (width 0.5) (layer "F.Cu") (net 1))
 (segment (start 136.38 87.199373) (end 133.420627 87.199373) (width 0.5) (layer "F.Cu") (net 1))
 (segment (start 137.10352 77.89648) (end 152.116922 77.89648) (width 0.5) (layer "F.Cu") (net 1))
 (via (at 142 93) (size 0.85) (drill 0.4) (layers "F.Cu" "B.Cu") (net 1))
 (segment (start 147.42534 99.0875) (end 147.42534 97.0875) (width 0.5) (layer "B.Cu") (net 1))
 (segment (start 151.0625 97) (end 147.51284 97) (width 0.5) (layer "B.Cu") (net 1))
 (segment (start 155.486766 81.563234) (end 155.783676 81.563234) (width 0.5) (layer "B.Cu") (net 1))
 (segment (start 147.51284 97) (end 147.42534 97.0875) (width 0.5) (layer "B.Cu") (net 1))
 (segment (start 142 93) (end 147 93) (width 0.5) (layer "B.Cu") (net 1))
 (segment (start 151.7 85.35) (end 155.486766 81.563234) (width 0.5) (layer "B.Cu") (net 1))
 (segment (start 147 93) (end 147.42534 93.42534) (width 0.5) (layer "B.Cu") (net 1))
 (segment (start 147.42534 93.42534) (end 147.42534 97.0875) (width 0.5) (layer "B.Cu") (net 1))
 (segment (start 151.7 87.85) (end 151.7 85.35) (width 0.5) (layer "B.Cu") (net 1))
 (segment (start 127.2125 108.2125) (end 128 108.2125) (width 0.5) (layer "B.Cu") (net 7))
 (segment (start 153 90) (end 154 89) (width 0.5) (layer "B.Cu") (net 7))
 (segment (start 149.438213 85.438213) (end 150 86) (width 0.5) (layer "B.Cu") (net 7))
 (segment (start 135.694373 90.425) (end 132 90.425) (width 0.5) (layer "B.Cu") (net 7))
 (segment (start 146.556323 85.438213) (end 149.438213 85.438213) (width 0.5) (layer "B.Cu") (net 7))
 (segment (start 127.9125 97.0875) (end 125 100) (width 0.5) (layer "B.Cu") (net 7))
 (segment (start 124 89) (end 130.575 89) (width 0.5) (layer "B.Cu") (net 7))
 (segment (start 133.33784 107) (end 133.42534 107.0875) (width 0.254) (layer "B.Cu") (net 7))
 (segment (start 151 90) (end 151 95.0625) (width 0.5) (layer "B.Cu") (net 7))
 (segment (start 138.92 87.199373) (end 135.694373 90.425) (width 0.5) (layer "B.Cu") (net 7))
 (segment (start 154 89) (end 154 87.85) (width 0.5) (layer "B.Cu") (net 7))
 (segment (start 128 108.2125) (end 129.2125 107) (width 0.254) (layer "B.Cu") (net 7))
 (segment (start 150 89) (end 151 90) (width 0.5) (layer "B.Cu") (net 7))
 (segment (start 133.42534 97.0875) (end 133.42534 92.694033) (width 0.5) (layer "B.Cu") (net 7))
 (segment (start 129.2125 107) (end 133.33784 107) (width 0.254) (layer "B.Cu") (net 7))
 (segment (start 138.92 87.199373) (end 140.68116 85.438213) (width 0.5) (layer "B.Cu") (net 7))
 (segment (start 133.42534 92.694033) (end 135.694373 90.425) (width 0.5) (layer "B.Cu") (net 7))
 (segment (start 151 90) (end 153 90) (width 0.5) (layer "B.Cu") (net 7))
 (segment (start 140.68116 85.438213) (end 146.556323 85.438213) (width 0.5) (layer "B.Cu") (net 7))
 (segment (start 125 106) (end 127.2125 108.2125) (width 0.5) (layer "B.Cu") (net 7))
 (segment (start 125 100) (end 125 106) (width 0.5) (layer "B.Cu") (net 7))
 (segment (start 150 86) (end 150 89) (width 0.5) (layer "B.Cu") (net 7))
 (segment (start 133.42534 97.0875) (end 127.9125 97.0875) (width 0.5) (layer "B.Cu") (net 7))
 (segment (start 130.575 89) (end 132 90.425) (width 0.5) (layer "B.Cu") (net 7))
 (segment (start 151 95.0625) (end 152.9375 97) (width 0.5) (layer "B.Cu") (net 7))
 (segment (start 141.46 88.46) (end 141.46 87.199373) (width 0.254) (layer "F.Cu") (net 9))
 (segment (start 144 91) (end 141.46 88.46) (width 0.254) (layer "F.Cu") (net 9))
 (segment (start 142 105) (end 144 103) (width 0.254) (layer "F.Cu") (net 9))
 (segment (start 144 103) (end 144 91) (width 0.254) (layer "F.Cu") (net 9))
 (via (at 142 105) (size 0.85) (drill 0.4) (layers "F.Cu" "B.Cu") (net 9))
 (segment (start 145 90) (end 146.556323 88.443677) (width 0.5) (layer "B.Cu") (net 9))
 (segment (start 141.46 88.46) (end 143 90) (width 0.5) (layer "B.Cu") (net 9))
 (segment (start 147.42534 107.0875) (end 144.0875 107.0875) (width 0.254) (layer "B.Cu") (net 9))
 (segment (start 143 90) (end 145 90) (width 0.5) (layer "B.Cu") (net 9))
 (segment (start 146.556323 88.443677) (end 146.556323 87.088213) (width 0.5) (layer "B.Cu") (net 9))
 (segment (start 141.46 87.199373) (end 141.46 88.46) (width 0.5) (layer "B.Cu") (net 9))
 (segment (start 144.0875 107.0875) (end 142 105) (width 0.254) (layer "B.Cu") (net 9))
 (segment (start 153.140442 84) (end 150.703676 81.563234) (width 0.254) (layer "F.Cu") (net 6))
 (segment (start 156.139166 84) (end 153.140442 84) (width 0.254) (layer "F.Cu") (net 6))
 (segment (start 156.805511 96.49248) (end 156.805511 84.666345) (width 0.254) (layer "F.Cu") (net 6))
 (segment (start 156.297991 104.702009) (end 156.297991 97) (width 0.254) (layer "F.Cu") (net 6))
 (segment (start 156.297991 97) (end 156.805511 96.49248) (width 0.254) (layer "F.Cu") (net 6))
 (segment (start 156.805511 84.666345) (end 156.139166 84) (width 0.254) (layer "F.Cu") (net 6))
 (segment (start 152 109) (end 156.297991 104.702009) (width 0.254) (layer "F.Cu") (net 6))
 (via (at 152 109) (size 0.85) (drill 0.4) (layers "F.Cu" "B.Cu") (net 6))
 (segment (start 147.42534 109.0875) (end 151.9125 109.0875) (width 0.254) (layer "B.Cu") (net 6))
 (segment (start 151.9125 109.0875) (end 152 109) (width 0.254) (layer "B.Cu") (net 6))
 (segment (start 157.79848 106.20152) (end 153 111) (width 0.254) (layer "F.Cu") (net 5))
 (segment (start 157.79848 84.79848) (end 157.79848 106.20152) (width 0.254) (layer "F.Cu") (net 5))
 (segment (start 156.49248 83.49248) (end 157.79848 84.79848) (width 0.254) (layer "F.Cu") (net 5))
 (segment (start 155.172922 83.49248) (end 156.49248 83.49248) (width 0.254) (layer "F.Cu") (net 5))
 (segment (start 153.243676 81.563234) (end 155.172922 83.49248) (width 0.254) (layer "F.Cu") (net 5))
 (via (at 153 111) (size 0.85) (drill 0.4) (layers "F.Cu" "B.Cu") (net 5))
 (segment (start 153 111) (end 147.51284 111) (width 0.254) (layer "B.Cu") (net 5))
 (segment (start 147.51284 111) (end 147.42534 111.0875) (width 0.254) (layer "B.Cu") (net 5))
 (segment (start 126 102) (end 124.175 102) (width 0.254) (layer "F.Cu") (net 3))
 (segment (start 124.175 102) (end 124 102.175) (width 0.254) (layer "F.Cu") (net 3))
 (via (at 126 102) (size 0.85) (drill 0.4) (layers "F.Cu" "B.Cu") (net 3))
 (segment (start 133.42534 105.0875) (end 129.0875 105.0875) (width 0.254) (layer "B.Cu") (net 3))
 (segment (start 129.0875 105.0875) (end 126 102) (width 0.254) (layer "B.Cu") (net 3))
 (segment (start 135 105) (end 130 110) (width 0.254) (layer "F.Cu") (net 4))
 (segment (start 139 105) (end 135 105) (width 0.254) (layer "F.Cu") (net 4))
 (segment (start 134 89) (end 134 94) (width 0.254) (layer "F.Cu") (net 4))
 (segment (start 134 94) (end 139 99) (width 0.254) (layer "F.Cu") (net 4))
 (via (at 139 99) (size 0.85) (drill 0.4) (layers "F.Cu" "B.Cu") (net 4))
 (via (at 130 110) (size 0.85) (drill 0.4) (layers "F.Cu" "B.Cu") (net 4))
 (via (at 134 89) (size 0.85) (drill 0.4) (layers "F.Cu" "B.Cu") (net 4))
 (via (at 139 105) (size 0.85) (drill 0.4) (layers "F.Cu" "B.Cu") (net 4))
 (segment (start 140.9125 100.9125) (end 139 99) (width 0.254) (layer "B.Cu") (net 4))
 (segment (start 129.7875 109.7875) (end 130 110) (width 0.254) (layer "B.Cu") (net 4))
 (segment (start 147.42534 103.0875) (end 140.9125 103.0875) (width 0.254) (layer "B.Cu") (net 4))
 (segment (start 140.9125 103.0875) (end 139 105) (width 0.254) (layer "B.Cu") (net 4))
 (segment (start 130.25 83.25) (end 134 87) (width 0.254) (layer "B.Cu") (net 4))
 (segment (start 128 109.7875) (end 129.7875 109.7875) (width 0.254) (layer "B.Cu") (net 4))
 (segment (start 140.9125 103.0875) (end 140.9125 100.9125) (width 0.254) (layer "B.Cu") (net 4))
 (segment (start 134 87) (end 134 89) (width 0.254) (layer "B.Cu") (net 4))
 (segment (start 123.75 83.25) (end 130.25 83.25) (width 0.254) (layer "B.Cu") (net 4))
 (segment (start 150 84) (end 151 85) (width 0.5) (layer "F.Cu") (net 11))
 (segment (start 151 85) (end 156 85) (width 0.5) (layer "F.Cu") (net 11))
 (segment (start 143.5 82.75) (end 145.75 82.75) (width 0.5) (layer "F.Cu") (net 11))
 (segment (start 147 84) (end 150 84) (width 0.5) (layer "F.Cu") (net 11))
 (segment (start 145.75 82.75) (end 147 84) (width 0.5) (layer "F.Cu") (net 11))
 (via (at 156 85) (size 0.85) (drill 0.4) (layers "F.Cu" "B.Cu") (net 11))
 (segment (start 156 87.55) (end 156.3 87.85) (width 0.5) (layer "B.Cu") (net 11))
 (segment (start 156 85) (end 153.95 85) (width 0.5) (layer "B.Cu") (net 11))
 (segment (start 156 85) (end 156 87.55) (width 0.5) (layer "B.Cu") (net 11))
 (segment (start 139 101) (end 132 94) (width 0.5) (layer "F.Cu") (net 8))
 (segment (start 142 101) (end 139 101) (width 0.5) (layer "F.Cu") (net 8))
 (via (at 132 94) (size 0.85) (drill 0.4) (layers "F.Cu" "B.Cu") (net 8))
 (via (at 142 101) (size 0.85) (drill 0.4) (layers "F.Cu" "B.Cu") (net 8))
 (segment (start 147.33784 101) (end 147.42534 101.0875) (width 0.5) (layer "B.Cu") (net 8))
 (segment (start 142 101) (end 147.33784 101) (width 0.5) (layer "B.Cu") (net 8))
 (segment (start 132 92) (end 132 94) (width 0.5) (layer "B.Cu") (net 8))
 (segment (start 129.54 91.54) (end 130 92) (width 0.5) (layer "B.Cu") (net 8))
 (segment (start 130 92) (end 132 92) (width 0.5) (layer "B.Cu") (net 8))
 (segment (start 124 91.54) (end 129.54 91.54) (width 0.5) (layer "B.Cu") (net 8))
 (segment (start 145 78) (end 145.85 78.85) (width 0.254) (layer "B.Cu") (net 14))
 (segment (start 145.85 78.85) (end 145.85 80) (width 0.254) (layer "B.Cu") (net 14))
 (segment (start 135 78) (end 145 78) (width 0.254) (layer "B.Cu") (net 14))
 (segment (start 134.15 78.85) (end 135 78) (width 0.254) (layer "B.Cu") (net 14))
 (segment (start 134.15 80) (end 134.15 78.85) (width 0.254) (layer "B.Cu") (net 14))
 (segment (start 146 90) (end 147 90) (width 0.5) (layer "F.Cu") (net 10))
 (segment (start 144 88) (end 146 90) (width 0.5) (layer "F.Cu") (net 10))
 (segment (start 147 90) (end 151 94) (width 0.5) (layer "F.Cu") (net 10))
 (segment (start 151 94) (end 151 103) (width 0.5) (layer "F.Cu") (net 10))
 (segment (start 144 87.199373) (end 144 88) (width 0.5) (layer "F.Cu") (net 10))
 (via (at 151 103) (size 0.85) (drill 0.4) (layers "F.Cu" "B.Cu") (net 10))
 (via (at 147 90) (size 0.85) (drill 0.4) (layers "F.Cu" "B.Cu") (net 10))
 (segment (start 151 104) (end 149.9125 105.0875) (width 0.5) (layer "B.Cu") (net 10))
 (segment (start 148.51575 87.075933) (end 148.51575 88.48425) (width 0.5) (layer "B.Cu") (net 10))
 (segment (start 148.51575 88.48425) (end 147 90) (width 0.5) (layer "B.Cu") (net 10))
 (segment (start 149.9125 105.0875) (end 147.42534 105.0875) (width 0.5) (layer "B.Cu") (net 10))
 (segment (start 151 104) (end 151 103) (width 0.5) (layer "B.Cu") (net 10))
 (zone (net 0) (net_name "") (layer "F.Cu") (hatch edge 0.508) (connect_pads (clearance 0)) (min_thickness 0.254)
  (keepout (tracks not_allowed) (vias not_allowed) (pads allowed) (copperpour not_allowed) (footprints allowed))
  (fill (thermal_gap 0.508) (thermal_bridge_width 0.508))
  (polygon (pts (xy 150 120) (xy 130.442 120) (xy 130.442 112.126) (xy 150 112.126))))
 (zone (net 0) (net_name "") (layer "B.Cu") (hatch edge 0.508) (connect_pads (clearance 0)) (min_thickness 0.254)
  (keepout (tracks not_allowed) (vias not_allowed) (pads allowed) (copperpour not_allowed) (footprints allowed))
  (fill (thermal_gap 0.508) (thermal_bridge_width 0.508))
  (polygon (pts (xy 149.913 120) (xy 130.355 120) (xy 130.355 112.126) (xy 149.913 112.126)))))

